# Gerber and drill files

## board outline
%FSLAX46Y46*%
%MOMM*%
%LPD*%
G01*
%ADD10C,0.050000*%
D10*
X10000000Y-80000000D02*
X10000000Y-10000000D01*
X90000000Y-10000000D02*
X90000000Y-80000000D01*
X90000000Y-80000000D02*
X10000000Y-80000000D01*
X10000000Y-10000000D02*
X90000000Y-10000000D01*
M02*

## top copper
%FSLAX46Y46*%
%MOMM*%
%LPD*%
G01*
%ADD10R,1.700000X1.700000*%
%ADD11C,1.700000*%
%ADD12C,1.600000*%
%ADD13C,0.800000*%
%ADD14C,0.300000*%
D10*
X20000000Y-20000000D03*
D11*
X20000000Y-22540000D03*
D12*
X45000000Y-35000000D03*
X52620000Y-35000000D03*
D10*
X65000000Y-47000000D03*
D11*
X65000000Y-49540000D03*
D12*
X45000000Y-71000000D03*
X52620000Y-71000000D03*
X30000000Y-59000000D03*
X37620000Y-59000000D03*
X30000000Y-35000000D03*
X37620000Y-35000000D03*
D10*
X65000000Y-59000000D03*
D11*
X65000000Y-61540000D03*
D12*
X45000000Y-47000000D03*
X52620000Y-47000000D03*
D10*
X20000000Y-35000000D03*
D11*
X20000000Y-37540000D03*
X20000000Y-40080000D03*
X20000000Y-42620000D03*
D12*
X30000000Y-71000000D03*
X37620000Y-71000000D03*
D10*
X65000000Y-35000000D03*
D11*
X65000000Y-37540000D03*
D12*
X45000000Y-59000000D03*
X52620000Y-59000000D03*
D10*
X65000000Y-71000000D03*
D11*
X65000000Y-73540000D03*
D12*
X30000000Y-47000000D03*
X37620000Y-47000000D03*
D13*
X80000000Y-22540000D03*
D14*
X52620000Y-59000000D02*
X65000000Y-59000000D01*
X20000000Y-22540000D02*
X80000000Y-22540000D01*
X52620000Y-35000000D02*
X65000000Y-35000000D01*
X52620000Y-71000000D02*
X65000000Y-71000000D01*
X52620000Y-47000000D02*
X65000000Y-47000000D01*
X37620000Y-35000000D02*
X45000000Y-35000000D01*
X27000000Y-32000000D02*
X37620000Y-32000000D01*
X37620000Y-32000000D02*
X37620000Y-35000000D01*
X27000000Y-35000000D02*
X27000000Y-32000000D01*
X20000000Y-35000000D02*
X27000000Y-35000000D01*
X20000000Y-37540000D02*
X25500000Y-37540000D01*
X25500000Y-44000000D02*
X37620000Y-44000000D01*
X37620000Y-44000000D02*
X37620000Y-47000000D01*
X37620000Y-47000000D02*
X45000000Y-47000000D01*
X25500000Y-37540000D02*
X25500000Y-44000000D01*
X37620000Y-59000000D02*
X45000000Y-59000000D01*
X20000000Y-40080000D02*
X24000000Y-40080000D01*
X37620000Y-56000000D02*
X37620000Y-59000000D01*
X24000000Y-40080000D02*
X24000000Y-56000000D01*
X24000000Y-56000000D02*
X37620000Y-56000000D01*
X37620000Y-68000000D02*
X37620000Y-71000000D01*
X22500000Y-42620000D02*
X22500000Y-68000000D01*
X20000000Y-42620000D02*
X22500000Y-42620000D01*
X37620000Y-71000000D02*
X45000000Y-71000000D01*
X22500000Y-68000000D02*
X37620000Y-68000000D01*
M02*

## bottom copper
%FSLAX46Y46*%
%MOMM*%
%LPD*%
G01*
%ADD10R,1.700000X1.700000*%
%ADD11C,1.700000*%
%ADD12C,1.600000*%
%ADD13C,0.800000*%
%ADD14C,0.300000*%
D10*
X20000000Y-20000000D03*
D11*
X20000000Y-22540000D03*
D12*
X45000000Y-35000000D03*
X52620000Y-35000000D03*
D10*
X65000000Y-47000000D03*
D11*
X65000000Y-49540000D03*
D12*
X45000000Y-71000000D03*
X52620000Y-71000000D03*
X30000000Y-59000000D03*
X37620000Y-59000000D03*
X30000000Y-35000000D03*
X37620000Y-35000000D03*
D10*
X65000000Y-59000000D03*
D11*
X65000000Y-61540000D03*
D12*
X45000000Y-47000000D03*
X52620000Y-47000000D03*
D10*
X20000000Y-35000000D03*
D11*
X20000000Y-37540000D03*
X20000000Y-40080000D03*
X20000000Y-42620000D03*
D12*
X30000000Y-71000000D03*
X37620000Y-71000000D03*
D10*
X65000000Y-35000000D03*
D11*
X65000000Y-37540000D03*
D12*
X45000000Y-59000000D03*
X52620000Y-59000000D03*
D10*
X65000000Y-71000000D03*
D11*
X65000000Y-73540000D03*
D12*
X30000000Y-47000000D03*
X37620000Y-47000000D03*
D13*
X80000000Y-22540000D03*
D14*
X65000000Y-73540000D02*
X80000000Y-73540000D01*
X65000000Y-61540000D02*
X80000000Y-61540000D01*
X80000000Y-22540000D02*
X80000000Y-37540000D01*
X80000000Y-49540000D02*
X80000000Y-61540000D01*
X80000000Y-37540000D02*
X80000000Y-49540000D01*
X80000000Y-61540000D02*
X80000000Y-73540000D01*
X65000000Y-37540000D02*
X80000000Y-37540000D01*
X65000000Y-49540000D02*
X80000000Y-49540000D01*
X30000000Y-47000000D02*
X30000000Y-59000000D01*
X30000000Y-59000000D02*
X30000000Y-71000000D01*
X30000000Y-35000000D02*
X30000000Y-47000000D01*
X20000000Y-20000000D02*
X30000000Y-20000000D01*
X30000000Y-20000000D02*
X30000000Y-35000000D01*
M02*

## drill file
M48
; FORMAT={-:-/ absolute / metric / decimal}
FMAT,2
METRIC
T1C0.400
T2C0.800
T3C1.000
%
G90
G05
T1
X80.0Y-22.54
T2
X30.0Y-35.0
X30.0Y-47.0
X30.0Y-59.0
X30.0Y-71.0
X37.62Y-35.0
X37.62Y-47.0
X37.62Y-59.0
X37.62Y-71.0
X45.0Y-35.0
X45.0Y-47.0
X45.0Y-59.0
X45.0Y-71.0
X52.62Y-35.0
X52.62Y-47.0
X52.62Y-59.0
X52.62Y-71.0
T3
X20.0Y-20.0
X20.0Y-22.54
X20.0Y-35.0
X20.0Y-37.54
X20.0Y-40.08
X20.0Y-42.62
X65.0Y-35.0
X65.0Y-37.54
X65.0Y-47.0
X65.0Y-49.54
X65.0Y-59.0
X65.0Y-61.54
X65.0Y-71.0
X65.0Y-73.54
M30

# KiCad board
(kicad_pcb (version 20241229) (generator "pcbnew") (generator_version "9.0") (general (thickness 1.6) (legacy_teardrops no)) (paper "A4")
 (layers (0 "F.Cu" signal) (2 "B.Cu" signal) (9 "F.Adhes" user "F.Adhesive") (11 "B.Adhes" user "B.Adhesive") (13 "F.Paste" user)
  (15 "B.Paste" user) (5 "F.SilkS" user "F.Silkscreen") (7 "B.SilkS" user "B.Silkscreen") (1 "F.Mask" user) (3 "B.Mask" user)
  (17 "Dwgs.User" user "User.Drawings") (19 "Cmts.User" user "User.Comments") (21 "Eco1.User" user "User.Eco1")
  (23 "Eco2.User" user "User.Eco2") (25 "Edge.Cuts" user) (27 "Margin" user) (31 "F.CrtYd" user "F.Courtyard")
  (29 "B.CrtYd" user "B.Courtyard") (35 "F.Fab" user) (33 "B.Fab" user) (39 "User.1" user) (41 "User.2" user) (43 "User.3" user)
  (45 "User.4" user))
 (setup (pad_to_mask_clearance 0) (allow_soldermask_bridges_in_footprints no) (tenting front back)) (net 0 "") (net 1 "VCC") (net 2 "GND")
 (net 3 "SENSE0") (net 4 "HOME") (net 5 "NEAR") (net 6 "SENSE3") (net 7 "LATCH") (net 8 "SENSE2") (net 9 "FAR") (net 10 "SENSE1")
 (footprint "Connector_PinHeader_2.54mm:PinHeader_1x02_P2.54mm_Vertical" (layer "F.Cu") (at 20 20)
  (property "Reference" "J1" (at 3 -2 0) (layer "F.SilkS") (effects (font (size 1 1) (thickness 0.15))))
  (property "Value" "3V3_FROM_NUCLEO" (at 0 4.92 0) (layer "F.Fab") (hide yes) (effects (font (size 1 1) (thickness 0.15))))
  (pad "1" thru_hole rect (at 0 0) (size 1.7 1.7) (drill 1) (layers "*.Cu" "*.Mask") (remove_unused_layers no) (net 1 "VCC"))
  (pad "2" thru_hole circle (at 0 2.54) (size 1.7 1.7) (drill 1) (layers "*.Cu" "*.Mask") (remove_unused_layers no) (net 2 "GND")))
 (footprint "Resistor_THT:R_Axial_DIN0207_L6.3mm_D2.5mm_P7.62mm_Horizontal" (layer "F.Cu") (at 45 35)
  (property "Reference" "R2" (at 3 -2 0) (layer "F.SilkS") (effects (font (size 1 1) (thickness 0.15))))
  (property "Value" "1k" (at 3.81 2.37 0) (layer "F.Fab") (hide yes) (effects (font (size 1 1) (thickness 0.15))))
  (pad "1" thru_hole circle (at 0 0) (size 1.6 1.6) (drill 0.8) (layers "*.Cu" "*.Mask") (remove_unused_layers no) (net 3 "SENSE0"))
  (pad "2" thru_hole circle (at 7.62 0) (size 1.6 1.6) (drill 0.8) (layers "*.Cu" "*.Mask") (remove_unused_layers no) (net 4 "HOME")))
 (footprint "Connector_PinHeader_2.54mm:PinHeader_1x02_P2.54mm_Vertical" (layer "F.Cu") (at 65 47)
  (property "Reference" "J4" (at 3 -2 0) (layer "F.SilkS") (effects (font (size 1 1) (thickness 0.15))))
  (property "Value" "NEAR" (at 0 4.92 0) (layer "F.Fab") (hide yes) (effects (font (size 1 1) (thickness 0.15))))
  (pad "1" thru_hole rect (at 0 0) (size 1.7 1.7) (drill 1) (layers "*.Cu" "*.Mask") (remove_unused_layers no) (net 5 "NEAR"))
  (pad "2" thru_hole circle (at 0 2.54) (size 1.7 1.7) (drill 1) (layers "*.Cu" "*.Mask") (remove_unused_layers no) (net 2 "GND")))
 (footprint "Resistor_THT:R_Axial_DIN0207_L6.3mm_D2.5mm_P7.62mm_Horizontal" (layer "F.Cu") (at 45 71)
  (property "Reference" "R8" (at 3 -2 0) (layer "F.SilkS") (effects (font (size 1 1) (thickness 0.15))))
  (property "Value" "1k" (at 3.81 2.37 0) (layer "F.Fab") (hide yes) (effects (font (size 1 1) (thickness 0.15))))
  (pad "1" thru_hole circle (at 0 0) (size 1.6 1.6) (drill 0.8) (layers "*.Cu" "*.Mask") (remove_unused_layers no) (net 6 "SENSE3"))
  (pad "2" thru_hole circle (at 7.62 0) (size 1.6 1.6) (drill 0.8) (layers "*.Cu" "*.Mask") (remove_unused_layers no) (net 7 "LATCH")))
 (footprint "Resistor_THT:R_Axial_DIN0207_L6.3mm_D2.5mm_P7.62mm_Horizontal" (layer "F.Cu") (at 30 59)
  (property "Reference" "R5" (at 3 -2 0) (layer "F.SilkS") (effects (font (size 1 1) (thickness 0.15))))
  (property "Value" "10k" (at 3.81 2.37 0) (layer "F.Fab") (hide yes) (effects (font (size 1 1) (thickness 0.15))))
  (pad "1" thru_hole circle (at 0 0) (size 1.6 1.6) (drill 0.8) (layers "*.Cu" "*.Mask") (remove_unused_layers no) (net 1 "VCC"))
  (pad "2" thru_hole circle (at 7.62 0) (size 1.6 1.6) (drill 0.8) (layers "*.Cu" "*.Mask") (remove_unused_layers no) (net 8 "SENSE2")))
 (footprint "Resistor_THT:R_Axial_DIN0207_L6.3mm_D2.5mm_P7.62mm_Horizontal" (layer "F.Cu") (at 30 35)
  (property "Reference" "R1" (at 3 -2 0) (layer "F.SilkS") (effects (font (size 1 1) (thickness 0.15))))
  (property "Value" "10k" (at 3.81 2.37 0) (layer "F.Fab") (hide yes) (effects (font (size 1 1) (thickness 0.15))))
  (pad "1" thru_hole circle (at 0 0) (size 1.6 1.6) (drill 0.8) (layers "*.Cu" "*.Mask") (remove_unused_layers no) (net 1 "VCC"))
  (pad "2" thru_hole circle (at 7.62 0) (size 1.6 1.6) (drill 0.8) (layers "*.Cu" "*.Mask") (remove_unused_layers no) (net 3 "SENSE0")))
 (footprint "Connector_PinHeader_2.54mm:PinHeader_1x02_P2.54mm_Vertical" (layer "F.Cu") (at 65 59)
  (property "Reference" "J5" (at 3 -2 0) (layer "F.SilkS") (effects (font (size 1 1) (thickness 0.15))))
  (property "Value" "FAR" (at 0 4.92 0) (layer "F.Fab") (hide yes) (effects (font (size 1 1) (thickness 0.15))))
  (pad "1" thru_hole rect (at 0 0) (size 1.7 1.7) (drill 1) (layers "*.Cu" "*.Mask") (remove_unused_layers no) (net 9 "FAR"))
  (pad "2" thru_hole circle (at 0 2.54) (size 1.7 1.7) (drill 1) (layers "*.Cu" "*.Mask") (remove_unused_layers no) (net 2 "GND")))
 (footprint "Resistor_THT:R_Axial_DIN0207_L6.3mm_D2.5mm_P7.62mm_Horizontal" (layer "F.Cu") (at 45 47)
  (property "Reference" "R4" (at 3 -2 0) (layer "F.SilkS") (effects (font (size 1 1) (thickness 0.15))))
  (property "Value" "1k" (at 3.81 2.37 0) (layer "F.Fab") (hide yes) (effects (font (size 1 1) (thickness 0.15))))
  (pad "1" thru_hole circle (at 0 0) (size 1.6 1.6) (drill 0.8) (layers "*.Cu" "*.Mask") (remove_unused_layers no) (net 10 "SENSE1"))
  (pad "2" thru_hole circle (at 7.62 0) (size 1.6 1.6) (drill 0.8) (layers "*.Cu" "*.Mask") (remove_unused_layers no) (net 5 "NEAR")))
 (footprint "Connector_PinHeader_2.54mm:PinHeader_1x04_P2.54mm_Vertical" (layer "F.Cu") (at 20 35)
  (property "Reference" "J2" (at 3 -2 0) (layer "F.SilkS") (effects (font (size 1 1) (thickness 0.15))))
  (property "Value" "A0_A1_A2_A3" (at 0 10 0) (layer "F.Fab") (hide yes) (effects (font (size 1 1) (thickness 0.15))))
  (pad "1" thru_hole rect (at 0 0) (size 1.7 1.7) (drill 1) (layers "*.Cu" "*.Mask") (remove_unused_layers no) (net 3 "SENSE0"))
  (pad "2" thru_hole circle (at 0 2.54) (size 1.7 1.7) (drill 1) (layers "*.Cu" "*.Mask") (remove_unused_layers no) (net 10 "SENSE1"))
  (pad "3" thru_hole circle (at 0 5.08) (size 1.7 1.7) (drill 1) (layers "*.Cu" "*.Mask") (remove_unused_layers no) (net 8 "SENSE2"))
  (pad "4" thru_hole circle (at 0 7.62) (size 1.7 1.7) (drill 1) (layers "*.Cu" "*.Mask") (remove_unused_layers no) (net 6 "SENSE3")))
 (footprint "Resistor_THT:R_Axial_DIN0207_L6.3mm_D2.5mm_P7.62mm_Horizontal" (layer "F.Cu") (at 30 71)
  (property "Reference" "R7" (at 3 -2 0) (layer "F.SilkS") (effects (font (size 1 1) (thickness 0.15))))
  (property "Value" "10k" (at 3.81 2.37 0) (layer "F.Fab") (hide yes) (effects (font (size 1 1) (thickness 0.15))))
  (pad "1" thru_hole circle (at 0 0) (size 1.6 1.6) (drill 0.8) (layers "*.Cu" "*.Mask") (remove_unused_layers no) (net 1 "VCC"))
  (pad "2" thru_hole circle (at 7.62 0) (size 1.6 1.6) (drill 0.8) (layers "*.Cu" "*.Mask") (remove_unused_layers no) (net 6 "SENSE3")))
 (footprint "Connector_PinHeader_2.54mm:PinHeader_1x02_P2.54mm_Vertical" (layer "F.Cu") (at 65 35)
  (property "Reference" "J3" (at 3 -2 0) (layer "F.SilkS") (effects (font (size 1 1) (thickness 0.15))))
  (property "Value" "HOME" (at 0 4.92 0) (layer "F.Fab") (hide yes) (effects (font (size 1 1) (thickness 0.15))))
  (pad "1" thru_hole rect (at 0 0) (size 1.7 1.7) (drill 1) (layers "*.Cu" "*.Mask") (remove_unused_layers no) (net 4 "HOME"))
  (pad "2" thru_hole circle (at 0 2.54) (size 1.7 1.7) (drill 1) (layers "*.Cu" "*.Mask") (remove_unused_layers no) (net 2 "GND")))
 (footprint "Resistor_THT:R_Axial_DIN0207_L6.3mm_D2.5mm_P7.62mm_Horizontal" (layer "F.Cu") (at 45 59)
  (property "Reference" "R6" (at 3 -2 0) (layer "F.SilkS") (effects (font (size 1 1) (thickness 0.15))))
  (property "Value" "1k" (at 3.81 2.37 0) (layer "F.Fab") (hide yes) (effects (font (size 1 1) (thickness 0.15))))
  (pad "1" thru_hole circle (at 0 0) (size 1.6 1.6) (drill 0.8) (layers "*.Cu" "*.Mask") (remove_unused_layers no) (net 8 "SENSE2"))
  (pad "2" thru_hole circle (at 7.62 0) (size 1.6 1.6) (drill 0.8) (layers "*.Cu" "*.Mask") (remove_unused_layers no) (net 9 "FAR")))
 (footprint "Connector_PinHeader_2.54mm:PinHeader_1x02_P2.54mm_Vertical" (layer "F.Cu") (at 65 71)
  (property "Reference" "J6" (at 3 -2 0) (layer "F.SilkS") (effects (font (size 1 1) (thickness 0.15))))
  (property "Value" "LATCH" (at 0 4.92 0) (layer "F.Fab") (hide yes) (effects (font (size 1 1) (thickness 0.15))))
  (pad "1" thru_hole rect (at 0 0) (size 1.7 1.7) (drill 1) (layers "*.Cu" "*.Mask") (remove_unused_layers no) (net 7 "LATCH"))
  (pad "2" thru_hole circle (at 0 2.54) (size 1.7 1.7) (drill 1) (layers "*.Cu" "*.Mask") (remove_unused_layers no) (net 2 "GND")))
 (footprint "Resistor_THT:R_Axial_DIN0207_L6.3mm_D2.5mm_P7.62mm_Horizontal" (layer "F.Cu") (at 30 47)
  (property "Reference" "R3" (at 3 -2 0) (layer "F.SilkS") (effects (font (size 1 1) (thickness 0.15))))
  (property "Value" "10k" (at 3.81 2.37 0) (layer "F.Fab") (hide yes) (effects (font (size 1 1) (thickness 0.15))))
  (pad "1" thru_hole circle (at 0 0) (size 1.6 1.6) (drill 0.8) (layers "*.Cu" "*.Mask") (remove_unused_layers no) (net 1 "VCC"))
  (pad "2" thru_hole circle (at 7.62 0) (size 1.6 1.6) (drill 0.8) (layers "*.Cu" "*.Mask") (remove_unused_layers no) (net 10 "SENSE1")))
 (gr_line (start 10 80) (end 10 10) (stroke (width 0.05) (type default)) (layer "Edge.Cuts"))
 (gr_line (start 90 10) (end 90 80) (stroke (width 0.05) (type default)) (layer "Edge.Cuts"))
 (gr_line (start 90 80) (end 10 80) (stroke (width 0.05) (type default)) (layer "Edge.Cuts"))
 (gr_line (start 10 10) (end 90 10) (stroke (width 0.05) (type default)) (layer "Edge.Cuts"))
 (segment (start 52.62 59) (end 65 59) (width 0.3) (layer "F.Cu") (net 9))
 (segment (start 20 22.54) (end 80 22.54) (width 0.3) (layer "F.Cu") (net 2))
 (via (at 80 22.54) (size 0.8) (drill 0.4) (layers "F.Cu" "B.Cu") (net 2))
 (segment (start 65 73.54) (end 80 73.54) (width 0.3) (layer "B.Cu") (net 2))
 (segment (start 65 61.54) (end 80 61.54) (width 0.3) (layer "B.Cu") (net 2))
 (segment (start 80 22.54) (end 80 37.54) (width 0.3) (layer "B.Cu") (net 2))
 (segment (start 80 49.54) (end 80 61.54) (width 0.3) (layer "B.Cu") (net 2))
 (segment (start 80 37.54) (end 80 49.54) (width 0.3) (layer "B.Cu") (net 2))
 (segment (start 80 61.54) (end 80 73.54) (width 0.3) (layer "B.Cu") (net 2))
 (segment (start 65 37.54) (end 80 37.54) (width 0.3) (layer "B.Cu") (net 2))
 (segment (start 65 49.54) (end 80 49.54) (width 0.3) (layer "B.Cu") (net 2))
 (segment (start 52.62 35) (end 65 35) (width 0.3) (layer "F.Cu") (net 4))
 (segment (start 52.62 71) (end 65 71) (width 0.3) (layer "F.Cu") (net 7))
 (segment (start 52.62 47) (end 65 47) (width 0.3) (layer "F.Cu") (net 5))
 (segment (start 37.62 35) (end 45 35) (width 0.3) (layer "F.Cu") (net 3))
 (segment (start 27 32) (end 37.62 32) (width 0.3) (layer "F.Cu") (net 3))
 (segment (start 37.62 32) (end 37.62 35) (width 0.3) (layer "F.Cu") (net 3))
 (segment (start 27 35) (end 27 32) (width 0.3) (layer "F.Cu") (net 3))
 (segment (start 20 35) (end 27 35) (width 0.3) (layer "F.Cu") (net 3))
 (segment (start 20 37.54) (end 25.5 37.54) (width 0.3) (layer "F.Cu") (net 10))
 (segment (start 25.5 44) (end 37.62 44) (width 0.3) (layer "F.Cu") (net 10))
 (segment (start 37.62 44) (end 37.62 47) (width 0.3) (layer "F.Cu") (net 10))
 (segment (start 37.62 47) (end 45 47) (width 0.3) (layer "F.Cu") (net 10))
 (segment (start 25.5 37.54) (end 25.5 44) (width 0.3) (layer "F.Cu") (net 10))
 (segment (start 37.62 59) (end 45 59) (width 0.3) (layer "F.Cu") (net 8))
 (segment (start 20 40.08) (end 24 40.08) (width 0.3) (layer "F.Cu") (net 8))
 (segment (start 37.62 56) (end 37.62 59) (width 0.3) (layer "F.Cu") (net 8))
 (segment (start 24 40.08) (end 24 56) (width 0.3) (layer "F.Cu") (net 8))
 (segment (start 24 56) (end 37.62 56) (width 0.3) (layer "F.Cu") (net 8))
 (segment (start 37.62 68) (end 37.62 71) (width 0.3) (layer "F.Cu") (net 6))
 (segment (start 22.5 42.62) (end 22.5 68) (width 0.3) (layer "F.Cu") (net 6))
 (segment (start 20 42.62) (end 22.5 42.62) (width 0.3) (layer "F.Cu") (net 6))
 (segment (start 37.62 71) (end 45 71) (width 0.3) (layer "F.Cu") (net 6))
 (segment (start 22.5 68) (end 37.62 68) (width 0.3) (layer "F.Cu") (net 6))
 (segment (start 30 47) (end 30 59) (width 0.3) (layer "B.Cu") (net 1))
 (segment (start 30 59) (end 30 71) (width 0.3) (layer "B.Cu") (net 1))
 (segment (start 30 35) (end 30 47) (width 0.3) (layer "B.Cu") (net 1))
 (segment (start 20 20) (end 30 20) (width 0.3) (layer "B.Cu") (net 1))
 (segment (start 30 20) (end 30 35) (width 0.3) (layer "B.Cu") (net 1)))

